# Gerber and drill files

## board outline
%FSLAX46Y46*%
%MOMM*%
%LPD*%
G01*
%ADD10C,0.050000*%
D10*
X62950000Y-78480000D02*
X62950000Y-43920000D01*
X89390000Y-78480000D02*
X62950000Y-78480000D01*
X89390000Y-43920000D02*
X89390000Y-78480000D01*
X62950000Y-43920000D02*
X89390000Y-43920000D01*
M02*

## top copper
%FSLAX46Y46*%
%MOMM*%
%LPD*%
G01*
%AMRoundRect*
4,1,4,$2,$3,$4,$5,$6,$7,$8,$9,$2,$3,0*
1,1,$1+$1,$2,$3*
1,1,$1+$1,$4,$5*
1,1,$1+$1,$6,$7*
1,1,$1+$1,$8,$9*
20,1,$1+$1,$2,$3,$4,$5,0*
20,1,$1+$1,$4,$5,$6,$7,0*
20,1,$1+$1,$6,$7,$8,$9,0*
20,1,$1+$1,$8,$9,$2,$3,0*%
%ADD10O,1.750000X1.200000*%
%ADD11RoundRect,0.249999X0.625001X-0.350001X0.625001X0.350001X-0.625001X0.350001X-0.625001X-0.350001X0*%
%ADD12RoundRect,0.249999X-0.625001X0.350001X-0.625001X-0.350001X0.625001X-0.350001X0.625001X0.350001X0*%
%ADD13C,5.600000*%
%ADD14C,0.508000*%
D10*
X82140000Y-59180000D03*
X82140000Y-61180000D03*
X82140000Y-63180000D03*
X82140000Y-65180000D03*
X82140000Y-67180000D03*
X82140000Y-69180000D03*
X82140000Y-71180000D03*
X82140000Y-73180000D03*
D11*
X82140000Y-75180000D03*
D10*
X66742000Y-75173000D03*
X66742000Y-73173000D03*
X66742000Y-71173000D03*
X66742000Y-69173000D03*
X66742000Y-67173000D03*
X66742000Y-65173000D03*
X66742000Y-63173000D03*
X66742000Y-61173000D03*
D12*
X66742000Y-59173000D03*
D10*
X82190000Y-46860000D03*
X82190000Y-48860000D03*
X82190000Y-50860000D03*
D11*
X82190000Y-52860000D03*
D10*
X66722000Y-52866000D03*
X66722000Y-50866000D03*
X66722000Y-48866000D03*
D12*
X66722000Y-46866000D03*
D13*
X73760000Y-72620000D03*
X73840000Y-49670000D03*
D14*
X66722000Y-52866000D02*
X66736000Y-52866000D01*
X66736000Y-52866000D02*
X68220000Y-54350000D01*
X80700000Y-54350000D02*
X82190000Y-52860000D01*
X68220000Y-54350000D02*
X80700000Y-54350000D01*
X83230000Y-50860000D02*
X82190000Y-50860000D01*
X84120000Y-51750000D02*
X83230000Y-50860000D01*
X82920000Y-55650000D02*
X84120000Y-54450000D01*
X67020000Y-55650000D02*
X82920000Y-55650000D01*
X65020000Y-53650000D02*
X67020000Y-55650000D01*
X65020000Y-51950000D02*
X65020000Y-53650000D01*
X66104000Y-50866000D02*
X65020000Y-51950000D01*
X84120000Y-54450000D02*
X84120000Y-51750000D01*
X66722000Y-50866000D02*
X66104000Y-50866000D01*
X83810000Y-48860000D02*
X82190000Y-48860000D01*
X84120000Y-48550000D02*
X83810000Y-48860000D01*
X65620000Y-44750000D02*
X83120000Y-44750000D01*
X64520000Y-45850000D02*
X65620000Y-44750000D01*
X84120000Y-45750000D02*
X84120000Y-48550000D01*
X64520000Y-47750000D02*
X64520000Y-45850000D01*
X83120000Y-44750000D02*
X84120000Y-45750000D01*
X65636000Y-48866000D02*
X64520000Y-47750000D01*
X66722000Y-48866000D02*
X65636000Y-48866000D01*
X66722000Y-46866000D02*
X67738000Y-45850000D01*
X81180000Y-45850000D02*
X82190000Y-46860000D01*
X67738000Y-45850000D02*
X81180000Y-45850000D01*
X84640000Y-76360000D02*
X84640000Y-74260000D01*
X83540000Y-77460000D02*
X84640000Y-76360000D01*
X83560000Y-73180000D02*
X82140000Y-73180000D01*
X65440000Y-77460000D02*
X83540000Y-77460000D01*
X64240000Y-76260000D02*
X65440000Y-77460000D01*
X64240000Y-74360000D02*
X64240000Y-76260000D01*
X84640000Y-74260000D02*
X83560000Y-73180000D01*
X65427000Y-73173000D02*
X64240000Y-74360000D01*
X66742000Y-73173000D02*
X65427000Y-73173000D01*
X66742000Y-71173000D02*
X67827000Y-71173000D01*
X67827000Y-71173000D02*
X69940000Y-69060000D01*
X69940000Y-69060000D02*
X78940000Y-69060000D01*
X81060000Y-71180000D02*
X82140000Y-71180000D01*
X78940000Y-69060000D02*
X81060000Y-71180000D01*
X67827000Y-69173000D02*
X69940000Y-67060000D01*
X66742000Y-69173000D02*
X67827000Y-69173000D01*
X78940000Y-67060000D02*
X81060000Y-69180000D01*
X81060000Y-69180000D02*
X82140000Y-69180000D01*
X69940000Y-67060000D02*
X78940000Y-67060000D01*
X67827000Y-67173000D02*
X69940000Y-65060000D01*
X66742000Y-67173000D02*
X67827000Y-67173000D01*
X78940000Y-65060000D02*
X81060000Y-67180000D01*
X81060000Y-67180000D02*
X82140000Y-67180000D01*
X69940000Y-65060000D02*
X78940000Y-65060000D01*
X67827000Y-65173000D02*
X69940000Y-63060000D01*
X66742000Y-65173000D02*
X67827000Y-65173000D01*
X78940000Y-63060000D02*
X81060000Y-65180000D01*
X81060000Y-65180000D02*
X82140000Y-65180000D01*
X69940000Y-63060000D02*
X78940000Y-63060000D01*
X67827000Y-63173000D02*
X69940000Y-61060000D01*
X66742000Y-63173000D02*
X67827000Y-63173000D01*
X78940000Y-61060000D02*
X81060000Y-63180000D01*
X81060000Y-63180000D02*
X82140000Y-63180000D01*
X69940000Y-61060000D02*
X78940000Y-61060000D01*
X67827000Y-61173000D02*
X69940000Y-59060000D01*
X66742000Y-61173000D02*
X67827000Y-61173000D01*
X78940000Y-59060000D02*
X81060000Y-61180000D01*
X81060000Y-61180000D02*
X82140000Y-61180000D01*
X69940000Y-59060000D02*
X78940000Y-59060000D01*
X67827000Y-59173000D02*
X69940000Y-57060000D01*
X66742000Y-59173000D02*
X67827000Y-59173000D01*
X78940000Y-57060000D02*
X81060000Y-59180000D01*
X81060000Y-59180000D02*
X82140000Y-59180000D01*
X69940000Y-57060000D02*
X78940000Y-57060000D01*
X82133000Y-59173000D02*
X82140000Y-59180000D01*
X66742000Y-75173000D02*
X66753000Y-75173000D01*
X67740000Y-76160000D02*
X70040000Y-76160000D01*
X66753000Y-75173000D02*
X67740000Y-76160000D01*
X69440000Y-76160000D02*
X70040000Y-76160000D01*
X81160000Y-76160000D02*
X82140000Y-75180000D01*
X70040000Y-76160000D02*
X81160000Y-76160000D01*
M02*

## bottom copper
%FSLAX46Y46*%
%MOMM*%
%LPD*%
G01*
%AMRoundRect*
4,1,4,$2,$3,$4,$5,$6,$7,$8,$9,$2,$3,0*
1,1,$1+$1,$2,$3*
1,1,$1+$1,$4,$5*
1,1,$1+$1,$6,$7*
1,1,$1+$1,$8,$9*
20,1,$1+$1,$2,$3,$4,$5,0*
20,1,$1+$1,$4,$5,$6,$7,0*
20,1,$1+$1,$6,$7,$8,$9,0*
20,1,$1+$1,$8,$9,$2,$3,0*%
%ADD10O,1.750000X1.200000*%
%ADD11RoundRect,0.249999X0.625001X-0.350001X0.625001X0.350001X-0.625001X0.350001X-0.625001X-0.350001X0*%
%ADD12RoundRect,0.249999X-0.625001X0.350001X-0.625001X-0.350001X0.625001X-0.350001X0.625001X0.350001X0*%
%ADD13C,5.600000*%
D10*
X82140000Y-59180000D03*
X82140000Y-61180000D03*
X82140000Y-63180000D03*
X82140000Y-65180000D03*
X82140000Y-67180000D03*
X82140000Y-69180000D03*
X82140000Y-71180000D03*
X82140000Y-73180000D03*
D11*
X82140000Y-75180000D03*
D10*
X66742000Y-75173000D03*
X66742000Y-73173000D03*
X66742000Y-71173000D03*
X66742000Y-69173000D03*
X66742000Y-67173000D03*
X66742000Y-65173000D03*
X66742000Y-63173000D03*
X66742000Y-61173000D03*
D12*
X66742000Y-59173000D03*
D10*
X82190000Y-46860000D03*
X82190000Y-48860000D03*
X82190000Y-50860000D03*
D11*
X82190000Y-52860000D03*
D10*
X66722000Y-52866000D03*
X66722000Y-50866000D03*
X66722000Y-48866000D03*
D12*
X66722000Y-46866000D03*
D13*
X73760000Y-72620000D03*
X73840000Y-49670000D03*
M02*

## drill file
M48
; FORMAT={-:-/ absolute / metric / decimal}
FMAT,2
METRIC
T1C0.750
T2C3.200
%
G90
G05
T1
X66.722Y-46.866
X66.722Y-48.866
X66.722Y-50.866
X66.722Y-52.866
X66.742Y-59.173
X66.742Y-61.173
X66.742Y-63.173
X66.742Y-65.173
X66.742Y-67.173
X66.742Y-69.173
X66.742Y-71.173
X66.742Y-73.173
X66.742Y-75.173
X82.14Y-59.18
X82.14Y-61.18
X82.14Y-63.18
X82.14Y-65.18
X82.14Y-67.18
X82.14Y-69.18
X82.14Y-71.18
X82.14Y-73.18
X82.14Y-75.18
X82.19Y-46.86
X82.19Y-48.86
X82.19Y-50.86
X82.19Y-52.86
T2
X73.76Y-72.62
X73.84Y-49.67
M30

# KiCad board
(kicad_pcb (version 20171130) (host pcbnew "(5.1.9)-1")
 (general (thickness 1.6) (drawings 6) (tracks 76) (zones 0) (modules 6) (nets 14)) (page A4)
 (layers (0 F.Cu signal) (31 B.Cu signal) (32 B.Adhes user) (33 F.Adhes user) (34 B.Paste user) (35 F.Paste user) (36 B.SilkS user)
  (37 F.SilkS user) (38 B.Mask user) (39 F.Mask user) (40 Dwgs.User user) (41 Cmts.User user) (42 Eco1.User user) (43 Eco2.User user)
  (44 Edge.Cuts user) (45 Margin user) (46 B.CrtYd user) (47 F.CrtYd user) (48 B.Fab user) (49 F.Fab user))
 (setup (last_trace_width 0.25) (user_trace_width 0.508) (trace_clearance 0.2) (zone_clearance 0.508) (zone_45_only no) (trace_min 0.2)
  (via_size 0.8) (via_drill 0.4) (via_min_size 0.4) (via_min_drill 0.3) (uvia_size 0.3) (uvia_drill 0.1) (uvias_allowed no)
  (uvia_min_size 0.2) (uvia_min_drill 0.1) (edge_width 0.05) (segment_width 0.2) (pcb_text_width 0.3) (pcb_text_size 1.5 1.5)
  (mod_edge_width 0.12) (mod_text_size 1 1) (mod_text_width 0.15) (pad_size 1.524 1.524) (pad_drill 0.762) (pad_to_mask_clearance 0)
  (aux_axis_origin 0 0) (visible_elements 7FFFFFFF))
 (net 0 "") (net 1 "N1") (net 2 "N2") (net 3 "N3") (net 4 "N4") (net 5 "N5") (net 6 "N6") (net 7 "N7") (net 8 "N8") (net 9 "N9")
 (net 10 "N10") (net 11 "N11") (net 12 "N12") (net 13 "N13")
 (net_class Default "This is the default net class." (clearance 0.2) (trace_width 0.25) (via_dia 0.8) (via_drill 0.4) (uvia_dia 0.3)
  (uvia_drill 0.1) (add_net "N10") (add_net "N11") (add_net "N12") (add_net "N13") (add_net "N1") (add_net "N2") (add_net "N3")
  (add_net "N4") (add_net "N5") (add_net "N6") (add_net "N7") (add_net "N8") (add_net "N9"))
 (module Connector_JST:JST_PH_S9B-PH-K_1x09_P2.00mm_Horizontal (layer F.Cu) (at 82.14 75.18 90)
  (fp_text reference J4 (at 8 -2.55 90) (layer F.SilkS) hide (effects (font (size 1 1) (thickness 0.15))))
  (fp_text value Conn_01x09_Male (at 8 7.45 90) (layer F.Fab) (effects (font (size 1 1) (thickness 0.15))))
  (pad 9 thru_hole oval (at 16 0 90) (size 1.2 1.75) (drill 0.75) (layers *.Cu *.Mask) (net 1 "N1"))
  (pad 8 thru_hole oval (at 14 0 90) (size 1.2 1.75) (drill 0.75) (layers *.Cu *.Mask) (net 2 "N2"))
  (pad 7 thru_hole oval (at 12 0 90) (size 1.2 1.75) (drill 0.75) (layers *.Cu *.Mask) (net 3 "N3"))
  (pad 6 thru_hole oval (at 10 0 90) (size 1.2 1.75) (drill 0.75) (layers *.Cu *.Mask) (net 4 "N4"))
  (pad 5 thru_hole oval (at 8 0 90) (size 1.2 1.75) (drill 0.75) (layers *.Cu *.Mask) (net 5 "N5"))
  (pad 4 thru_hole oval (at 6 0 90) (size 1.2 1.75) (drill 0.75) (layers *.Cu *.Mask) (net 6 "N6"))
  (pad 3 thru_hole oval (at 4 0 90) (size 1.2 1.75) (drill 0.75) (layers *.Cu *.Mask) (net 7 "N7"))
  (pad 2 thru_hole oval (at 2 0 90) (size 1.2 1.75) (drill 0.75) (layers *.Cu *.Mask) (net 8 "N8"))
  (pad 1 thru_hole roundrect (at 0 0 90) (size 1.2 1.75) (drill 0.75) (layers *.Cu *.Mask) (roundrect_rratio 0.2083325) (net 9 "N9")))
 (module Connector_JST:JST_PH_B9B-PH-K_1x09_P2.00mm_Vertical (layer F.Cu) (at 66.742 59.173 270)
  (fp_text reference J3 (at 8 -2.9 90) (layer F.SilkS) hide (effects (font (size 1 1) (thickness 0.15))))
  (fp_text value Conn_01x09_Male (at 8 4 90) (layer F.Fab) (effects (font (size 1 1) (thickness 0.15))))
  (pad 9 thru_hole oval (at 16 0 270) (size 1.2 1.75) (drill 0.75) (layers *.Cu *.Mask) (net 9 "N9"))
  (pad 8 thru_hole oval (at 14 0 270) (size 1.2 1.75) (drill 0.75) (layers *.Cu *.Mask) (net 8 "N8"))
  (pad 7 thru_hole oval (at 12 0 270) (size 1.2 1.75) (drill 0.75) (layers *.Cu *.Mask) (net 7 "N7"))
  (pad 6 thru_hole oval (at 10 0 270) (size 1.2 1.75) (drill 0.75) (layers *.Cu *.Mask) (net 6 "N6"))
  (pad 5 thru_hole oval (at 8 0 270) (size 1.2 1.75) (drill 0.75) (layers *.Cu *.Mask) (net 5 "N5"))
  (pad 4 thru_hole oval (at 6 0 270) (size 1.2 1.75) (drill 0.75) (layers *.Cu *.Mask) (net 4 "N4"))
  (pad 3 thru_hole oval (at 4 0 270) (size 1.2 1.75) (drill 0.75) (layers *.Cu *.Mask) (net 3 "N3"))
  (pad 2 thru_hole oval (at 2 0 270) (size 1.2 1.75) (drill 0.75) (layers *.Cu *.Mask) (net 2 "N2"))
  (pad 1 thru_hole roundrect (at 0 0 270) (size 1.2 1.75) (drill 0.75) (layers *.Cu *.Mask) (roundrect_rratio 0.2083325) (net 1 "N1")))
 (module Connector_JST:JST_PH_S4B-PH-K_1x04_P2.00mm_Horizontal (layer F.Cu) (at 82.19 52.86 90)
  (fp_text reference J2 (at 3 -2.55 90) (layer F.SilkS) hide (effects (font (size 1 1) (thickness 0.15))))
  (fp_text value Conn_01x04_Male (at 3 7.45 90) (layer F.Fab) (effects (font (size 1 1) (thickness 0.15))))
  (pad 4 thru_hole oval (at 6 0 90) (size 1.2 1.75) (drill 0.75) (layers *.Cu *.Mask) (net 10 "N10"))
  (pad 3 thru_hole oval (at 4 0 90) (size 1.2 1.75) (drill 0.75) (layers *.Cu *.Mask) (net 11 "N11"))
  (pad 2 thru_hole oval (at 2 0 90) (size 1.2 1.75) (drill 0.75) (layers *.Cu *.Mask) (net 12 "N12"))
  (pad 1 thru_hole roundrect (at 0 0 90) (size 1.2 1.75) (drill 0.75) (layers *.Cu *.Mask) (roundrect_rratio 0.2083325) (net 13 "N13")))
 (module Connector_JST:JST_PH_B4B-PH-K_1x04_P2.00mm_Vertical (layer F.Cu) (at 66.722 46.866 270)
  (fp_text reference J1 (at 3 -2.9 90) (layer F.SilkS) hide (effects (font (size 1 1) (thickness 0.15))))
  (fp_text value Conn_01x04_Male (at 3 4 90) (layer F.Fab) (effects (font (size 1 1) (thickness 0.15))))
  (pad 4 thru_hole oval (at 6 0 270) (size 1.2 1.75) (drill 0.75) (layers *.Cu *.Mask) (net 13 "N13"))
  (pad 3 thru_hole oval (at 4 0 270) (size 1.2 1.75) (drill 0.75) (layers *.Cu *.Mask) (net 12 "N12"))
  (pad 2 thru_hole oval (at 2 0 270) (size 1.2 1.75) (drill 0.75) (layers *.Cu *.Mask) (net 11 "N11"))
  (pad 1 thru_hole roundrect (at 0 0 270) (size 1.2 1.75) (drill 0.75) (layers *.Cu *.Mask) (roundrect_rratio 0.2083325) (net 10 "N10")))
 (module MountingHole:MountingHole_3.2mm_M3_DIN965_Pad (layer F.Cu) (at 73.76 72.62)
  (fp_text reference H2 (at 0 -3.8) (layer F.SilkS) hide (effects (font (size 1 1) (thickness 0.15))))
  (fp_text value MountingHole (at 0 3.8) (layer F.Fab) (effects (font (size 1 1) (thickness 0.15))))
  (pad 1 thru_hole circle (at 0 0) (size 5.6 5.6) (drill 3.2) (layers *.Cu *.Mask)))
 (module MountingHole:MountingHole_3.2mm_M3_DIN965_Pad (layer F.Cu) (at 73.84 49.67)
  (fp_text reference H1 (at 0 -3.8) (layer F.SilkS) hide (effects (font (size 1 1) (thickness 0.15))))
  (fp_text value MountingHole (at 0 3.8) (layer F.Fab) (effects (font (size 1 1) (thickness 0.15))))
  (pad 1 thru_hole circle (at 0 0) (size 5.6 5.6) (drill 3.2) (layers *.Cu *.Mask)))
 (gr_line (start 62.95 78.48) (end 62.95 43.92) (layer Edge.Cuts) (width 0.05))
 (gr_line (start 89.39 78.48) (end 62.95 78.48) (layer Edge.Cuts) (width 0.05))
 (gr_line (start 89.39 43.92) (end 89.39 78.48) (layer Edge.Cuts) (width 0.05))
 (gr_line (start 62.95 43.92) (end 89.39 43.92) (layer Edge.Cuts) (width 0.05))
 (segment (start 66.722 52.866) (end 66.736 52.866) (width 0.508) (layer F.Cu) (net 13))
 (segment (start 66.736 52.866) (end 68.22 54.35) (width 0.508) (layer F.Cu) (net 13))
 (segment (start 80.7 54.35) (end 82.19 52.86) (width 0.508) (layer F.Cu) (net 13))
 (segment (start 68.22 54.35) (end 80.7 54.35) (width 0.508) (layer F.Cu) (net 13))
 (segment (start 83.23 50.86) (end 82.19 50.86) (width 0.508) (layer F.Cu) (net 12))
 (segment (start 84.12 51.75) (end 83.23 50.86) (width 0.508) (layer F.Cu) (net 12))
 (segment (start 82.92 55.65) (end 84.12 54.45) (width 0.508) (layer F.Cu) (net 12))
 (segment (start 67.02 55.65) (end 82.92 55.65) (width 0.508) (layer F.Cu) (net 12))
 (segment (start 65.02 53.65) (end 67.02 55.65) (width 0.508) (layer F.Cu) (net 12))
 (segment (start 65.02 51.95) (end 65.02 53.65) (width 0.508) (layer F.Cu) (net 12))
 (segment (start 66.104 50.866) (end 65.02 51.95) (width 0.508) (layer F.Cu) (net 12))
 (segment (start 84.12 54.45) (end 84.12 51.75) (width 0.508) (layer F.Cu) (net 12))
 (segment (start 66.722 50.866) (end 66.104 50.866) (width 0.508) (layer F.Cu) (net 12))
 (segment (start 83.81 48.86) (end 82.19 48.86) (width 0.508) (layer F.Cu) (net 11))
 (segment (start 84.12 48.55) (end 83.81 48.86) (width 0.508) (layer F.Cu) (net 11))
 (segment (start 65.62 44.75) (end 83.12 44.75) (width 0.508) (layer F.Cu) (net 11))
 (segment (start 64.52 45.85) (end 65.62 44.75) (width 0.508) (layer F.Cu) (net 11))
 (segment (start 84.12 45.75) (end 84.12 48.55) (width 0.508) (layer F.Cu) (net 11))
 (segment (start 64.52 47.75) (end 64.52 45.85) (width 0.508) (layer F.Cu) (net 11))
 (segment (start 83.12 44.75) (end 84.12 45.75) (width 0.508) (layer F.Cu) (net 11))
 (segment (start 65.636 48.866) (end 64.52 47.75) (width 0.508) (layer F.Cu) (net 11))
 (segment (start 66.722 48.866) (end 65.636 48.866) (width 0.508) (layer F.Cu) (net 11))
 (segment (start 66.722 46.866) (end 67.738 45.85) (width 0.508) (layer F.Cu) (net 10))
 (segment (start 81.18 45.85) (end 82.19 46.86) (width 0.508) (layer F.Cu) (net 10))
 (segment (start 67.738 45.85) (end 81.18 45.85) (width 0.508) (layer F.Cu) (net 10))
 (segment (start 84.64 76.36) (end 84.64 74.26) (width 0.508) (layer F.Cu) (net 8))
 (segment (start 83.54 77.46) (end 84.64 76.36) (width 0.508) (layer F.Cu) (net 8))
 (segment (start 83.56 73.18) (end 82.14 73.18) (width 0.508) (layer F.Cu) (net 8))
 (segment (start 65.44 77.46) (end 83.54 77.46) (width 0.508) (layer F.Cu) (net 8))
 (segment (start 64.24 76.26) (end 65.44 77.46) (width 0.508) (layer F.Cu) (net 8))
 (segment (start 64.24 74.36) (end 64.24 76.26) (width 0.508) (layer F.Cu) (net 8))
 (segment (start 84.64 74.26) (end 83.56 73.18) (width 0.508) (layer F.Cu) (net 8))
 (segment (start 65.427 73.173) (end 64.24 74.36) (width 0.508) (layer F.Cu) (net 8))
 (segment (start 66.742 73.173) (end 65.427 73.173) (width 0.508) (layer F.Cu) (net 8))
 (segment (start 66.742 71.173) (end 67.827 71.173) (width 0.508) (layer F.Cu) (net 7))
 (segment (start 67.827 71.173) (end 69.94 69.06) (width 0.508) (layer F.Cu) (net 7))
 (segment (start 69.94 69.06) (end 78.94 69.06) (width 0.508) (layer F.Cu) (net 7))
 (segment (start 81.06 71.18) (end 82.14 71.18) (width 0.508) (layer F.Cu) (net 7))
 (segment (start 78.94 69.06) (end 81.06 71.18) (width 0.508) (layer F.Cu) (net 7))
 (segment (start 67.827 69.173) (end 69.94 67.06) (width 0.508) (layer F.Cu) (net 6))
 (segment (start 66.742 69.173) (end 67.827 69.173) (width 0.508) (layer F.Cu) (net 6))
 (segment (start 78.94 67.06) (end 81.06 69.18) (width 0.508) (layer F.Cu) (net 6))
 (segment (start 81.06 69.18) (end 82.14 69.18) (width 0.508) (layer F.Cu) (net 6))
 (segment (start 69.94 67.06) (end 78.94 67.06) (width 0.508) (layer F.Cu) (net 6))
 (segment (start 67.827 67.173) (end 69.94 65.06) (width 0.508) (layer F.Cu) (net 5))
 (segment (start 66.742 67.173) (end 67.827 67.173) (width 0.508) (layer F.Cu) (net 5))
 (segment (start 78.94 65.06) (end 81.06 67.18) (width 0.508) (layer F.Cu) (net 5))
 (segment (start 81.06 67.18) (end 82.14 67.18) (width 0.508) (layer F.Cu) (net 5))
 (segment (start 69.94 65.06) (end 78.94 65.06) (width 0.508) (layer F.Cu) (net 5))
 (segment (start 67.827 65.173) (end 69.94 63.06) (width 0.508) (layer F.Cu) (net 4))
 (segment (start 66.742 65.173) (end 67.827 65.173) (width 0.508) (layer F.Cu) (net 4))
 (segment (start 78.94 63.06) (end 81.06 65.18) (width 0.508) (layer F.Cu) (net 4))
 (segment (start 81.06 65.18) (end 82.14 65.18) (width 0.508) (layer F.Cu) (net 4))
 (segment (start 69.94 63.06) (end 78.94 63.06) (width 0.508) (layer F.Cu) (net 4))
 (segment (start 67.827 63.173) (end 69.94 61.06) (width 0.508) (layer F.Cu) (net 3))
 (segment (start 66.742 63.173) (end 67.827 63.173) (width 0.508) (layer F.Cu) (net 3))
 (segment (start 78.94 61.06) (end 81.06 63.18) (width 0.508) (layer F.Cu) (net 3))
 (segment (start 81.06 63.18) (end 82.14 63.18) (width 0.508) (layer F.Cu) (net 3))
 (segment (start 69.94 61.06) (end 78.94 61.06) (width 0.508) (layer F.Cu) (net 3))
 (segment (start 67.827 61.173) (end 69.94 59.06) (width 0.508) (layer F.Cu) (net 2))
 (segment (start 66.742 61.173) (end 67.827 61.173) (width 0.508) (layer F.Cu) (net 2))
 (segment (start 78.94 59.06) (end 81.06 61.18) (width 0.508) (layer F.Cu) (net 2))
 (segment (start 81.06 61.18) (end 82.14 61.18) (width 0.508) (layer F.Cu) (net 2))
 (segment (start 69.94 59.06) (end 78.94 59.06) (width 0.508) (layer F.Cu) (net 2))
 (segment (start 67.827 59.173) (end 69.94 57.06) (width 0.508) (layer F.Cu) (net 1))
 (segment (start 66.742 59.173) (end 67.827 59.173) (width 0.508) (layer F.Cu) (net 1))
 (segment (start 78.94 57.06) (end 81.06 59.18) (width 0.508) (layer F.Cu) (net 1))
 (segment (start 81.06 59.18) (end 82.14 59.18) (width 0.508) (layer F.Cu) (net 1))
 (segment (start 69.94 57.06) (end 78.94 57.06) (width 0.508) (layer F.Cu) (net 1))
 (segment (start 82.133 59.173) (end 82.14 59.18) (width 0.508) (layer F.Cu) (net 1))
 (segment (start 66.742 75.173) (end 66.753 75.173) (width 0.508) (layer F.Cu) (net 9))
 (segment (start 67.74 76.16) (end 70.04 76.16) (width 0.508) (layer F.Cu) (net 9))
 (segment (start 66.753 75.173) (end 67.74 76.16) (width 0.508) (layer F.Cu) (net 9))
 (segment (start 69.44 76.16) (end 70.04 76.16) (width 0.508) (layer F.Cu) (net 9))
 (segment (start 81.16 76.16) (end 82.14 75.18) (width 0.508) (layer F.Cu) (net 9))
 (segment (start 70.04 76.16) (end 81.16 76.16) (width 0.508) (layer F.Cu) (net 9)))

